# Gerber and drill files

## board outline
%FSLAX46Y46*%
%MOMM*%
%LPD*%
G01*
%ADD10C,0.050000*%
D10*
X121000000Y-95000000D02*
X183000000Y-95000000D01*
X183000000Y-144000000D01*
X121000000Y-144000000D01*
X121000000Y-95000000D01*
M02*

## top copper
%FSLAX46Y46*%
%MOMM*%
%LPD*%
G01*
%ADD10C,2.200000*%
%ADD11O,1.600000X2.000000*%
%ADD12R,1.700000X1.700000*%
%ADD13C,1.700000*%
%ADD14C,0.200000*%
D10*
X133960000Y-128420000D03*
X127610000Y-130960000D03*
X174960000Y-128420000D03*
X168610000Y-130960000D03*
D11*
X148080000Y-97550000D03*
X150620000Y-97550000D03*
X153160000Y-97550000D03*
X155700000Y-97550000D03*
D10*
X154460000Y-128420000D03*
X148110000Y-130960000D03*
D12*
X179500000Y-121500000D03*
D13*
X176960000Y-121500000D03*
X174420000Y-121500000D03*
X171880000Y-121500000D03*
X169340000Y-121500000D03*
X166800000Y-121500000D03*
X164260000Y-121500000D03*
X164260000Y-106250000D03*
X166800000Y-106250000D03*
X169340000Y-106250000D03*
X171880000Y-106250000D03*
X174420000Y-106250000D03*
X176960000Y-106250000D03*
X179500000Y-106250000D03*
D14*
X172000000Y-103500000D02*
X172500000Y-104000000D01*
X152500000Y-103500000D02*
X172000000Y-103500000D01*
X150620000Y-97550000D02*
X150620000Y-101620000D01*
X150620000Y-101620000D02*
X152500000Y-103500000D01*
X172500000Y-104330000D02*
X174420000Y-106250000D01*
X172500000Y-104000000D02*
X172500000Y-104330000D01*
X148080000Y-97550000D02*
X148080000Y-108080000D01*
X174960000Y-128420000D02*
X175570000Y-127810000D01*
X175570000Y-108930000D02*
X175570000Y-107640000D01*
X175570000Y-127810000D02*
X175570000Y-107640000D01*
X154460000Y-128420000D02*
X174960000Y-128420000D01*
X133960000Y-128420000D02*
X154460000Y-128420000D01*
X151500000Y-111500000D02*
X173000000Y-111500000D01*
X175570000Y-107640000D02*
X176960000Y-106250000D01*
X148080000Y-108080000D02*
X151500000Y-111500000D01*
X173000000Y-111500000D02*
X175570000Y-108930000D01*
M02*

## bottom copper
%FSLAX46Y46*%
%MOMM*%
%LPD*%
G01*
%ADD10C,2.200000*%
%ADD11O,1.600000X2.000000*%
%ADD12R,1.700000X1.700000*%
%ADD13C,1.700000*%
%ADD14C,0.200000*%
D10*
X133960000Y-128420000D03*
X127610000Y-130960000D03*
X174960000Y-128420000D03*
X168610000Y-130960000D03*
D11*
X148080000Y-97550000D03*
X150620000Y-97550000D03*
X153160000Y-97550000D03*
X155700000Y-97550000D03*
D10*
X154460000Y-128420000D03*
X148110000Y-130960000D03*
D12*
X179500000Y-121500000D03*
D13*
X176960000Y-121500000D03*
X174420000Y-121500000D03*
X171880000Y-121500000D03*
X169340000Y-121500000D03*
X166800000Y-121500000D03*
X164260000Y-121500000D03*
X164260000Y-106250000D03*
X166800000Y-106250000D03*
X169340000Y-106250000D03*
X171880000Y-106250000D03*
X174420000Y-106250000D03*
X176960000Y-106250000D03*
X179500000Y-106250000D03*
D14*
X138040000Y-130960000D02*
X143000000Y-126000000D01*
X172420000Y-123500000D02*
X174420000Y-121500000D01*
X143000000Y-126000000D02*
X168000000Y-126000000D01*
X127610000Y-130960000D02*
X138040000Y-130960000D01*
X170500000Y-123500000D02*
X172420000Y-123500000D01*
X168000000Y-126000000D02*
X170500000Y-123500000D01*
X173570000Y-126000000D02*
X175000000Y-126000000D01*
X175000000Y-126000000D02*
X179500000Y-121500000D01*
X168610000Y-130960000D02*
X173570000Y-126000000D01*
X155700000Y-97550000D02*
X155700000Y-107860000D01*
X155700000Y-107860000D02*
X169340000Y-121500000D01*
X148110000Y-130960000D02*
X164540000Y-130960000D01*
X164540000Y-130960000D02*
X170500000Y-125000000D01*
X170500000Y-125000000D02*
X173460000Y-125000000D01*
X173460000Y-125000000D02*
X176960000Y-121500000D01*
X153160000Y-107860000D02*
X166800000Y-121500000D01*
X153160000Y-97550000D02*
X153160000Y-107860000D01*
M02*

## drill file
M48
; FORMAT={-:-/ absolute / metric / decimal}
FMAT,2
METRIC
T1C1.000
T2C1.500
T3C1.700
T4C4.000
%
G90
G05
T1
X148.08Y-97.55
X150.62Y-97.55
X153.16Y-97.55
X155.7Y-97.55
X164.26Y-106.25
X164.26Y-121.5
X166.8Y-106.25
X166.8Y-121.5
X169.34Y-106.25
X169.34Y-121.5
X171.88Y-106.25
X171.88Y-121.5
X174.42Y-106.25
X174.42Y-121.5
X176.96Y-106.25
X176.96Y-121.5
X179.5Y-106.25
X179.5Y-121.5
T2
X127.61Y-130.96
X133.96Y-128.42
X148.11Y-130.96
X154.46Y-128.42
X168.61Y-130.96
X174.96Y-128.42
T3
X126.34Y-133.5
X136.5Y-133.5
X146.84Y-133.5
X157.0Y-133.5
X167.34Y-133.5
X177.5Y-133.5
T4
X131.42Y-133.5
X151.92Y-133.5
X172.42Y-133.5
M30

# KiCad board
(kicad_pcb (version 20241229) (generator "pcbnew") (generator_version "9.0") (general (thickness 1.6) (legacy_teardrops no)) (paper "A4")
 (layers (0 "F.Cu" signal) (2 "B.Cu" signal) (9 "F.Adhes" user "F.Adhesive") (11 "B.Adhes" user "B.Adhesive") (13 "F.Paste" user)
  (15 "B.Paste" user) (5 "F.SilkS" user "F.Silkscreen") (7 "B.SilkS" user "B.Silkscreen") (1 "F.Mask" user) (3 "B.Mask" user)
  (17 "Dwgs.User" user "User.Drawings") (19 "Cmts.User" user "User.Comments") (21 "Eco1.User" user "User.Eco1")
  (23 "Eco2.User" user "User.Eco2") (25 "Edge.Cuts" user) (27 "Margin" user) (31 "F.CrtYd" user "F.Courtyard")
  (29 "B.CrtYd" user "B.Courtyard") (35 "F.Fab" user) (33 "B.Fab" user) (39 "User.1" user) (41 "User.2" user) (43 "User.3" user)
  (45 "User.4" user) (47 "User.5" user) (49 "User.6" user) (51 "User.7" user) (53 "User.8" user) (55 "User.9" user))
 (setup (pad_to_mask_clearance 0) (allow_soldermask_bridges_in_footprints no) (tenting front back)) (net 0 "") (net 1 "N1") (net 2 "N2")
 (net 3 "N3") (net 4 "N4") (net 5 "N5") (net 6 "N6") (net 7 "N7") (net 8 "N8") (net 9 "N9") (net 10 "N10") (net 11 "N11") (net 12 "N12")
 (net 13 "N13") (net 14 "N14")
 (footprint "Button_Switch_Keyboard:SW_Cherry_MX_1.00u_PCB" (layer "F.Cu") (at 133.96 128.42)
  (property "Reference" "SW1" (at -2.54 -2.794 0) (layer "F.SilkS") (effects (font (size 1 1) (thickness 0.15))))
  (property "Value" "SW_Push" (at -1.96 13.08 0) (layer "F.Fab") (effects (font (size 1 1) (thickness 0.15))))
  (pad "" np_thru_hole circle (at -7.62 5.08) (size 1.7 1.7) (drill 1.7) (layers "*.Cu" "*.Mask"))
  (pad "" np_thru_hole circle (at -2.54 5.08) (size 4 4) (drill 4) (layers "*.Cu" "*.Mask"))
  (pad "" np_thru_hole circle (at 2.54 5.08) (size 1.7 1.7) (drill 1.7) (layers "*.Cu" "*.Mask"))
  (pad "1" thru_hole circle (at 0 0) (size 2.2 2.2) (drill 1.5) (layers "*.Cu" "*.Mask") (remove_unused_layers no) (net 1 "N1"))
  (pad "2" thru_hole circle (at -6.35 2.54) (size 2.2 2.2) (drill 1.5) (layers "*.Cu" "*.Mask") (remove_unused_layers no) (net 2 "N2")))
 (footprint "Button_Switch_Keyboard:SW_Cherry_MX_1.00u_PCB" (layer "F.Cu") (at 174.96 128.42)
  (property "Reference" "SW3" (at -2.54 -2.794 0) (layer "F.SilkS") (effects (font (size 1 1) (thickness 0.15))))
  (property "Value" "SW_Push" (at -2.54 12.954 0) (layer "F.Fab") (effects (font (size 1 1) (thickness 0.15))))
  (pad "" np_thru_hole circle (at -7.62 5.08) (size 1.7 1.7) (drill 1.7) (layers "*.Cu" "*.Mask"))
  (pad "" np_thru_hole circle (at -2.54 5.08) (size 4 4) (drill 4) (layers "*.Cu" "*.Mask"))
  (pad "" np_thru_hole circle (at 2.54 5.08) (size 1.7 1.7) (drill 1.7) (layers "*.Cu" "*.Mask"))
  (pad "1" thru_hole circle (at 0 0) (size 2.2 2.2) (drill 1.5) (layers "*.Cu" "*.Mask") (remove_unused_layers no) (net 1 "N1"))
  (pad "2" thru_hole circle (at -6.35 2.54) (size 2.2 2.2) (drill 1.5) (layers "*.Cu" "*.Mask") (remove_unused_layers no) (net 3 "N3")))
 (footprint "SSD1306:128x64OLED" (layer "F.Cu") (at 151.7 108.15)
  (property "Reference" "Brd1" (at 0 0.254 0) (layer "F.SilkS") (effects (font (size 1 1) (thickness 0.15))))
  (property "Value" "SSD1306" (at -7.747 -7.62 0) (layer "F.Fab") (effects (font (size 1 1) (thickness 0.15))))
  (pad "1" thru_hole oval (at -3.62 -10.6 90) (size 2 1.6) (drill 1) (layers "*.Cu" "*.Mask") (remove_unused_layers no) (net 1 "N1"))
  (pad "2" thru_hole oval (at -1.08 -10.6 90) (size 2 1.6) (drill 1) (layers "*.Cu" "*.Mask") (remove_unused_layers no) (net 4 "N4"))
  (pad "3" thru_hole oval (at 1.46 -10.6 90) (size 2 1.6) (drill 1) (layers "*.Cu" "*.Mask") (remove_unused_layers no) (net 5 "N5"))
  (pad "4" thru_hole oval (at 4 -10.6 90) (size 2 1.6) (drill 1) (layers "*.Cu" "*.Mask") (remove_unused_layers no) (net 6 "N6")))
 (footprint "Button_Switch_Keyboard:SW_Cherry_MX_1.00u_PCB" (layer "F.Cu") (at 154.46 128.42)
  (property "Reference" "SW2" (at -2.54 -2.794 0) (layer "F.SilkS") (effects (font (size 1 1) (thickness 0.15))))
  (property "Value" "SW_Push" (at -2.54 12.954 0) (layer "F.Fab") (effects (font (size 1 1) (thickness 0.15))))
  (pad "" np_thru_hole circle (at -7.62 5.08) (size 1.7 1.7) (drill 1.7) (layers "*.Cu" "*.Mask"))
  (pad "" np_thru_hole circle (at -2.54 5.08) (size 4 4) (drill 4) (layers "*.Cu" "*.Mask"))
  (pad "" np_thru_hole circle (at 2.54 5.08) (size 1.7 1.7) (drill 1.7) (layers "*.Cu" "*.Mask"))
  (pad "1" thru_hole circle (at 0 0) (size 2.2 2.2) (drill 1.5) (layers "*.Cu" "*.Mask") (remove_unused_layers no) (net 1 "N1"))
  (pad "2" thru_hole circle (at -6.35 2.54) (size 2.2 2.2) (drill 1.5) (layers "*.Cu" "*.Mask") (remove_unused_layers no) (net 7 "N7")))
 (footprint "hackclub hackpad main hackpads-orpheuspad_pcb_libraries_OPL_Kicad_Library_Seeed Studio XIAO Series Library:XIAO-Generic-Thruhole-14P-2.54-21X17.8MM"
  (layer "B.Cu") (at 171.88 113.875 90)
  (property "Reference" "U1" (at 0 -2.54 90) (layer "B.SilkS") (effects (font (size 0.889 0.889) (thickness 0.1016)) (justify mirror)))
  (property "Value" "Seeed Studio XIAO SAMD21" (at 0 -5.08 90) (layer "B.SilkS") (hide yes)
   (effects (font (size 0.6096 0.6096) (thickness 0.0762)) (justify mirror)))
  (pad "1" thru_hole rect (at -7.625 7.62 90) (size 1.7 1.7) (drill 1) (layers "*.Cu" "*.Mask") (remove_unused_layers no) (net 3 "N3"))
  (pad "2" thru_hole circle (at -7.625 5.08 90) (size 1.7 1.7) (drill 1) (layers "*.Cu" "*.Mask") (remove_unused_layers no) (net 7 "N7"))
  (pad "3" thru_hole circle (at -7.625 2.54 90) (size 1.7 1.7) (drill 1) (layers "*.Cu" "*.Mask") (remove_unused_layers no) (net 2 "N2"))
  (pad "4" thru_hole circle (at -7.625 0 90) (size 1.7 1.7) (drill 1) (layers "*.Cu" "*.Mask") (remove_unused_layers no) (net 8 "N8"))
  (pad "5" thru_hole circle (at -7.625 -2.54 90) (size 1.7 1.7) (drill 1) (layers "*.Cu" "*.Mask") (remove_unused_layers no) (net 6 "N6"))
  (pad "6" thru_hole circle (at -7.625 -5.08 270) (size 1.7 1.7) (drill 1) (layers "*.Cu" "*.Mask") (remove_unused_layers no) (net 5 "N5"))
  (pad "7" thru_hole circle (at -7.625 -7.62 90) (size 1.7 1.7) (drill 1) (layers "*.Cu" "*.Mask") (remove_unused_layers no) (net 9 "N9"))
  (pad "8" thru_hole circle (at 7.625 -7.62 90) (size 1.7 1.7) (drill 1) (layers "*.Cu" "*.Mask") (remove_unused_layers no) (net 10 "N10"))
  (pad "9" thru_hole circle (at 7.625 -5.08 90) (size 1.7 1.7) (drill 1) (layers "*.Cu" "*.Mask") (remove_unused_layers no) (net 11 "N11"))
  (pad "10" thru_hole circle (at 7.625 -2.54 90) (size 1.7 1.7) (drill 1) (layers "*.Cu" "*.Mask") (remove_unused_layers no) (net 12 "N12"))
  (pad "11" thru_hole circle (at 7.625 0 90) (size 1.7 1.7) (drill 1) (layers "*.Cu" "*.Mask") (remove_unused_layers no) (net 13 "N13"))
  (pad "12" thru_hole circle (at 7.625 2.54 90) (size 1.7 1.7) (drill 1) (layers "*.Cu" "*.Mask") (remove_unused_layers no) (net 4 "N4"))
  (pad "13" thru_hole circle (at 7.625 5.08 90) (size 1.7 1.7) (drill 1) (layers "*.Cu" "*.Mask") (remove_unused_layers no) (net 1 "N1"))
  (pad "14" thru_hole circle (at 7.625 7.62 90) (size 1.7 1.7) (drill 1) (layers "*.Cu" "*.Mask") (remove_unused_layers no) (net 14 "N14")))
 (gr_rect (start 121 95) (end 183 144) (stroke (width 0.05) (type default)) (fill no) (layer "Edge.Cuts"))
 (segment (start 138.04 130.96) (end 143 126) (width 0.2) (layer "B.Cu") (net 2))
 (segment (start 172.42 123.5) (end 174.42 121.5) (width 0.2) (layer "B.Cu") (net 2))
 (segment (start 143 126) (end 168 126) (width 0.2) (layer "B.Cu") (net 2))
 (segment (start 127.61 130.96) (end 138.04 130.96) (width 0.2) (layer "B.Cu") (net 2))
 (segment (start 170.5 123.5) (end 172.42 123.5) (width 0.2) (layer "B.Cu") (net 2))
 (segment (start 168 126) (end 170.5 123.5) (width 0.2) (layer "B.Cu") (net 2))
 (segment (start 172 103.5) (end 172.5 104) (width 0.2) (layer "F.Cu") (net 4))
 (segment (start 152.5 103.5) (end 172 103.5) (width 0.2) (layer "F.Cu") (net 4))
 (segment (start 150.62 97.55) (end 150.62 101.62) (width 0.2) (layer "F.Cu") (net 4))
 (segment (start 150.62 101.62) (end 152.5 103.5) (width 0.2) (layer "F.Cu") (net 4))
 (segment (start 172.5 104.33) (end 174.42 106.25) (width 0.2) (layer "F.Cu") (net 4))
 (segment (start 172.5 104) (end 172.5 104.33) (width 0.2) (layer "F.Cu") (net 4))
 (segment (start 173.57 126) (end 175 126) (width 0.2) (layer "B.Cu") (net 3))
 (segment (start 175 126) (end 179.5 121.5) (width 0.2) (layer "B.Cu") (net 3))
 (segment (start 168.61 130.96) (end 173.57 126) (width 0.2) (layer "B.Cu") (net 3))
 (segment (start 148.08 97.55) (end 148.08 108.08) (width 0.2) (layer "F.Cu") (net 1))
 (segment (start 174.96 128.42) (end 175.57 127.81) (width 0.2) (layer "F.Cu") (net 1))
 (segment (start 175.57 108.93) (end 175.57 107.64) (width 0.2) (layer "F.Cu") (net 1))
 (segment (start 175.57 127.81) (end 175.57 107.64) (width 0.2) (layer "F.Cu") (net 1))
 (segment (start 154.46 128.42) (end 174.96 128.42) (width 0.2) (layer "F.Cu") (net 1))
 (segment (start 133.96 128.42) (end 154.46 128.42) (width 0.2) (layer "F.Cu") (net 1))
 (segment (start 151.5 111.5) (end 173 111.5) (width 0.2) (layer "F.Cu") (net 1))
 (segment (start 175.57 107.64) (end 176.96 106.25) (width 0.2) (layer "F.Cu") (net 1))
 (segment (start 148.08 108.08) (end 151.5 111.5) (width 0.2) (layer "F.Cu") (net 1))
 (segment (start 173 111.5) (end 175.57 108.93) (width 0.2) (layer "F.Cu") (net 1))
 (segment (start 155.7 97.55) (end 155.7 107.86) (width 0.2) (layer "B.Cu") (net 6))
 (segment (start 155.7 107.86) (end 169.34 121.5) (width 0.2) (layer "B.Cu") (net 6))
 (segment (start 148.11 130.96) (end 164.54 130.96) (width 0.2) (layer "B.Cu") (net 7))
 (segment (start 164.54 130.96) (end 170.5 125) (width 0.2) (layer "B.Cu") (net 7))
 (segment (start 170.5 125) (end 173.46 125) (width 0.2) (layer "B.Cu") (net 7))
 (segment (start 173.46 125) (end 176.96 121.5) (width 0.2) (layer "B.Cu") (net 7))
 (segment (start 153.16 107.86) (end 166.8 121.5) (width 0.2) (layer "B.Cu") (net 5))
 (segment (start 153.16 97.55) (end 153.16 107.86) (width 0.2) (layer "B.Cu") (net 5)))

